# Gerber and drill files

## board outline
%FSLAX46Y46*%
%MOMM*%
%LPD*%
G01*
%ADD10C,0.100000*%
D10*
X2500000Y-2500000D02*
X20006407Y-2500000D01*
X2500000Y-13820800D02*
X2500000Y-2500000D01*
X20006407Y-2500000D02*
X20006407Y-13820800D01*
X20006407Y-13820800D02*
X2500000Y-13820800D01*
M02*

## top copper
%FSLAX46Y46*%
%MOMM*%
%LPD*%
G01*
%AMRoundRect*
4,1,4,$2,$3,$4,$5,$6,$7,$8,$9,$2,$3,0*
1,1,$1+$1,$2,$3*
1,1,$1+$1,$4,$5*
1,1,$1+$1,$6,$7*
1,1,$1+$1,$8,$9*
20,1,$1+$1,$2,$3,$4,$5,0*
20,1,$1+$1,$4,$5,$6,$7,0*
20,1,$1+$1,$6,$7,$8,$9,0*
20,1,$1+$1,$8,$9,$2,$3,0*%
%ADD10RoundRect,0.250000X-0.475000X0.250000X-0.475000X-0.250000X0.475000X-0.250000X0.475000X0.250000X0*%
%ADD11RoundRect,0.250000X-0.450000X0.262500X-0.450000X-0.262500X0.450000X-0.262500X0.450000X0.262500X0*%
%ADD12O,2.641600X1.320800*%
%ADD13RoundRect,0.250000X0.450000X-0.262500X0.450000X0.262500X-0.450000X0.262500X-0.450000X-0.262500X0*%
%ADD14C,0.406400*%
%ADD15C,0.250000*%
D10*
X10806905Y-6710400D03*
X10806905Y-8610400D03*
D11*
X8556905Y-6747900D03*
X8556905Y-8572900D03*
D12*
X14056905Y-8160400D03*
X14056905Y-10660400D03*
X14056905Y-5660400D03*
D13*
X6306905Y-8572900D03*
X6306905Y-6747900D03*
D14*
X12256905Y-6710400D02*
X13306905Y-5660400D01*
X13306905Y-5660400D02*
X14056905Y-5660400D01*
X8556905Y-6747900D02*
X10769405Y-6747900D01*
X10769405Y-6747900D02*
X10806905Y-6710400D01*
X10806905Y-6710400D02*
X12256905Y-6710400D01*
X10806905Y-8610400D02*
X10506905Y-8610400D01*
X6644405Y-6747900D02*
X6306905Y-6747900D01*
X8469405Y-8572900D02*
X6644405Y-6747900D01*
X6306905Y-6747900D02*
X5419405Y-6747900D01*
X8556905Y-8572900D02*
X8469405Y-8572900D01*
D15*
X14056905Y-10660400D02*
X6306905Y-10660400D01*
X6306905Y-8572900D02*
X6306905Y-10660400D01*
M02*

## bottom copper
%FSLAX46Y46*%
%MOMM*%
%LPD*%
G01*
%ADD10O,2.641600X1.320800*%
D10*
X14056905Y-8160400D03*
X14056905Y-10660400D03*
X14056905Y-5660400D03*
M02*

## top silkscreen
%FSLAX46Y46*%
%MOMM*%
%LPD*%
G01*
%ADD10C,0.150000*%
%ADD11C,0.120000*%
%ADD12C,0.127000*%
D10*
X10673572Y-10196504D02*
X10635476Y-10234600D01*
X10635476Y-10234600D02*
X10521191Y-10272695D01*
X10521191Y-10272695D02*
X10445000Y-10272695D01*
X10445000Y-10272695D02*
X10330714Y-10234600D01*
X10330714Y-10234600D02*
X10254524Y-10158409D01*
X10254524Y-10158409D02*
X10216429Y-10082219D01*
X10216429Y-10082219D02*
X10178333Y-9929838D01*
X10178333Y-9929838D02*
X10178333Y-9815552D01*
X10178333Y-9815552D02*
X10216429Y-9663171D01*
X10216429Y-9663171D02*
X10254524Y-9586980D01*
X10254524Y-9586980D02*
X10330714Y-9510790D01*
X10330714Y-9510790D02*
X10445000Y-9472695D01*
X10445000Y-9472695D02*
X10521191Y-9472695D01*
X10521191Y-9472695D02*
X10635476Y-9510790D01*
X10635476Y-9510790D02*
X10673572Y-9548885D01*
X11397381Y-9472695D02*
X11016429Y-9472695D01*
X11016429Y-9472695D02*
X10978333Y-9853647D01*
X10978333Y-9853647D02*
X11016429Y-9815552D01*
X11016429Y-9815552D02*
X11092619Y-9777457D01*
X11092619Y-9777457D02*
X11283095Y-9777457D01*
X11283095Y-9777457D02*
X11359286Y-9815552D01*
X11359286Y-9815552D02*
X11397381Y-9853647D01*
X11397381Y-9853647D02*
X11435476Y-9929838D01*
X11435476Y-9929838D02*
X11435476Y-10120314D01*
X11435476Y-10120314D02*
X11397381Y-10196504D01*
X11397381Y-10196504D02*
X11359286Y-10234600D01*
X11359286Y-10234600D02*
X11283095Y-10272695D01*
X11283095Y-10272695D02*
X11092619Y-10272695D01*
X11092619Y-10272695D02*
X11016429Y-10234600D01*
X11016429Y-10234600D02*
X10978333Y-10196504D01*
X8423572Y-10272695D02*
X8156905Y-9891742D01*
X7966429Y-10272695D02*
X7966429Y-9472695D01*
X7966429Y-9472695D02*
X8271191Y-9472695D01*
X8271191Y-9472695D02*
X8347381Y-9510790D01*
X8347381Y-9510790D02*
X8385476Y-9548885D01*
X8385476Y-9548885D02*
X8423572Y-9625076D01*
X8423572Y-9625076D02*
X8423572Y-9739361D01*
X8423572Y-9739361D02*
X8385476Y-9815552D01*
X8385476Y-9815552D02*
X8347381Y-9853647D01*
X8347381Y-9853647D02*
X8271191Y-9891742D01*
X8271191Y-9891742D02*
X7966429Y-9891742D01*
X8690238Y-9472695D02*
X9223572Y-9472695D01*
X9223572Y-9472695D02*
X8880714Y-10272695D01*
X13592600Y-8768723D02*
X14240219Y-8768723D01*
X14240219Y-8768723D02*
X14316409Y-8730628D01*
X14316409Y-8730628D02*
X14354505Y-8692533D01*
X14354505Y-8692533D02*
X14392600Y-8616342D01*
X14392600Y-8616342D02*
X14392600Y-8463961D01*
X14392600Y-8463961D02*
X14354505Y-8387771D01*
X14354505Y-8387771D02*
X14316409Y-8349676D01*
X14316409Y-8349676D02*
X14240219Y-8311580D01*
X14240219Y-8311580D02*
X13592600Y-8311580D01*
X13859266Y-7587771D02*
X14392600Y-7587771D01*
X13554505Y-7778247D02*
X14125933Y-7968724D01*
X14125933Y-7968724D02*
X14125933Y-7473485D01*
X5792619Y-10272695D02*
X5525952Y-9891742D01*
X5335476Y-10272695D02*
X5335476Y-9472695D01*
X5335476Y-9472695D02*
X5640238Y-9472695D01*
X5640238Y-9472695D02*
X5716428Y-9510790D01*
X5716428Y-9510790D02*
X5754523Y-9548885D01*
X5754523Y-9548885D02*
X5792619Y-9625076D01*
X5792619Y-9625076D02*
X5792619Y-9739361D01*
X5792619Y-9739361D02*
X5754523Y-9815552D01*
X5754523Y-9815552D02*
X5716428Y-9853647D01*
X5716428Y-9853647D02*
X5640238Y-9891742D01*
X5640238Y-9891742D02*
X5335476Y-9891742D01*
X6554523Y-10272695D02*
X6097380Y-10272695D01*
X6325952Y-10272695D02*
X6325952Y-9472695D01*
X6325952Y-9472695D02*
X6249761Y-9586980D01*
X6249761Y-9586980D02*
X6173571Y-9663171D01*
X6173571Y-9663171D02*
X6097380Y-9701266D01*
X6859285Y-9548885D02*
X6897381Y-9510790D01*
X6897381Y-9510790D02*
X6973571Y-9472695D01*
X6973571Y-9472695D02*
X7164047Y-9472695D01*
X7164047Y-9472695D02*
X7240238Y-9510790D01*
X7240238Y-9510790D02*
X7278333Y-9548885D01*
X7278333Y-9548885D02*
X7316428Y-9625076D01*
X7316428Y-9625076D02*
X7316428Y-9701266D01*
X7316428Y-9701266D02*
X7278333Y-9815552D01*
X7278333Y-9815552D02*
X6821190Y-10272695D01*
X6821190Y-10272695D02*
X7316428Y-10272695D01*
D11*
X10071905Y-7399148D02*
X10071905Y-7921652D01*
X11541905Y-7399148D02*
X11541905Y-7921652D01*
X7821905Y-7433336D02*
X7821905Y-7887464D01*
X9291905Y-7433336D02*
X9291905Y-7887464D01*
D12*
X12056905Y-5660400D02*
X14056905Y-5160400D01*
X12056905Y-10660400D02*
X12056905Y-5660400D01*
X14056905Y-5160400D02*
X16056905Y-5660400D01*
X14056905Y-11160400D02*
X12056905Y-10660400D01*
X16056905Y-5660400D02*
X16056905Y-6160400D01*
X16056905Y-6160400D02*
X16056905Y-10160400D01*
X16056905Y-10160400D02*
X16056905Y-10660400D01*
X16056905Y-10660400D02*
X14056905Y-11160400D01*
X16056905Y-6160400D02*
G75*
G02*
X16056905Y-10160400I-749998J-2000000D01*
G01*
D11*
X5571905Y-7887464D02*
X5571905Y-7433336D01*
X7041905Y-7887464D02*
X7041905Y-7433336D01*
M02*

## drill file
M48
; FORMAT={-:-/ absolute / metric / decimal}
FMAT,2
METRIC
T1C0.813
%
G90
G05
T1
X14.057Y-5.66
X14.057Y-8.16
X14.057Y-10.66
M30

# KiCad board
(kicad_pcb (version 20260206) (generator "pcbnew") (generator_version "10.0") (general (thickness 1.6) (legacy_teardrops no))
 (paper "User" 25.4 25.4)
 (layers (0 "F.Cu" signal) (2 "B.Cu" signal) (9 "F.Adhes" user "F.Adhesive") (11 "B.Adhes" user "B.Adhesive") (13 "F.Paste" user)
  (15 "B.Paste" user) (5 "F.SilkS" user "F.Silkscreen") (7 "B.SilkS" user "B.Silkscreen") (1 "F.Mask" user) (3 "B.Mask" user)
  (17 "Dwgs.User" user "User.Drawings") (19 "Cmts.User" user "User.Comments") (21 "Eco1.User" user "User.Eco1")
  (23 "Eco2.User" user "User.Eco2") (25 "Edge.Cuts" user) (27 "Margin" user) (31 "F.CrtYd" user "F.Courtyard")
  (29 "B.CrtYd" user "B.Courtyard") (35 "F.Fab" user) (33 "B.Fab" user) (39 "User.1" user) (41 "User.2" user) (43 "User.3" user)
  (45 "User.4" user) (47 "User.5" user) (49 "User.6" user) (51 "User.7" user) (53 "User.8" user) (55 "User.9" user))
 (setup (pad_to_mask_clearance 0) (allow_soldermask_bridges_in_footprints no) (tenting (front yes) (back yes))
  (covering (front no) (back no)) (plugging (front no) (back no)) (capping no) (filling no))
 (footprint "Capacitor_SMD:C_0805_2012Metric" (layer "F.Cu") (at 10.806905 7.6604 -90)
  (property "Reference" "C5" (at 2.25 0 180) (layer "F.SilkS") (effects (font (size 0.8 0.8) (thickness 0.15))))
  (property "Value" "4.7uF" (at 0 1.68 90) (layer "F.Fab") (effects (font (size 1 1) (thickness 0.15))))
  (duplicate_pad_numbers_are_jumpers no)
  (fp_line (start -0.261252 0.735) (end 0.261252 0.735) (stroke (width 0.12) (type solid)) (layer "F.SilkS"))
  (fp_line (start -0.261252 -0.735) (end 0.261252 -0.735) (stroke (width 0.12) (type solid)) (layer "F.SilkS"))
  (pad "1" smd roundrect (at -0.95 0 270) (size 1 1.45) (layers "F.Cu" "F.Mask" "F.Paste") (roundrect_rratio 0.25) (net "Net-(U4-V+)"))
  (pad "2" smd roundrect (at 0.95 0 270) (size 1 1.45) (layers "F.Cu" "F.Mask" "F.Paste") (roundrect_rratio 0.25) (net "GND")))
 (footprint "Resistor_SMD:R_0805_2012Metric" (layer "F.Cu") (at 8.556905 7.6604 -90)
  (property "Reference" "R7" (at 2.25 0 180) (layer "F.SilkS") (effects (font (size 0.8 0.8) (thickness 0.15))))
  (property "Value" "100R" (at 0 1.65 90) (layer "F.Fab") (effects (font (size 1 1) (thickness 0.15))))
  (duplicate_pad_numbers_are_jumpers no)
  (fp_line (start -0.227064 0.735) (end 0.227064 0.735) (stroke (width 0.12) (type solid)) (layer "F.SilkS"))
  (fp_line (start -0.227064 -0.735) (end 0.227064 -0.735) (stroke (width 0.12) (type solid)) (layer "F.SilkS"))
  (pad "1" smd roundrect (at -0.9125 0 270) (size 1.025 1.4) (layers "F.Cu" "F.Mask" "F.Paste") (roundrect_rratio 0.243902439)
   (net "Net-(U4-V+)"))
  (pad "2" smd roundrect (at 0.9125 0 270) (size 1.025 1.4) (layers "F.Cu" "F.Mask" "F.Paste") (roundrect_rratio 0.243902439) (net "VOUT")))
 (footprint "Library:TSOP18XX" (layer "F.Cu") (at 14.030305 8.1592 90)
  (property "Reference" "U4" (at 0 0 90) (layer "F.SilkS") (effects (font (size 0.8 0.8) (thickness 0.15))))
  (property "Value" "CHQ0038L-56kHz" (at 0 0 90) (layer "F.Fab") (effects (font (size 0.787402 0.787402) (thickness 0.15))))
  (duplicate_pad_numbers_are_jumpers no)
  (fp_line (start 2.4988 -1.9734) (end 2.9988 0.0266) (stroke (width 0.127) (type solid)) (layer "F.SilkS"))
  (fp_line (start -2.5012 -1.9734) (end 2.4988 -1.9734) (stroke (width 0.127) (type solid)) (layer "F.SilkS"))
  (fp_line (start 2.9988 0.0266) (end 2.4988 2.0266) (stroke (width 0.127) (type solid)) (layer "F.SilkS"))
  (fp_line (start -3.0012 0.0266) (end -2.5012 -1.9734) (stroke (width 0.127) (type solid)) (layer "F.SilkS"))
  (fp_line (start 2.4988 2.0266) (end 1.9988 2.0266) (stroke (width 0.127) (type solid)) (layer "F.SilkS"))
  (fp_line (start 1.9988 2.0266) (end -2.0012 2.0266) (stroke (width 0.127) (type solid)) (layer "F.SilkS"))
  (fp_line (start -2.0012 2.0266) (end -2.5012 2.0266) (stroke (width 0.127) (type solid)) (layer "F.SilkS"))
  (fp_line (start -2.5012 2.0266) (end -3.0012 0.0266) (stroke (width 0.127) (type solid)) (layer "F.SilkS"))
  (fp_arc (start 1.9988 2.0266) (mid -0.0012 3.412602) (end -2.0012 2.0266) (stroke (width 0.127) (type solid)) (layer "F.SilkS"))
  (pad "GND" thru_hole oval (at -0.0012 0.0266 90) (size 1.3208 2.6416) (drill 0.8128) (layers "*.Cu" "*.Mask") (remove_unused_layers no)
   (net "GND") (solder_mask_margin 0.102))
  (pad "OUT" thru_hole oval (at -2.5012 0.0266 90) (size 1.3208 2.6416) (drill 0.8128) (layers "*.Cu" "*.Mask") (remove_unused_layers no)
   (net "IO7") (solder_mask_margin 0.102))
  (pad "VCC" thru_hole oval (at 2.4988 0.0266 90) (size 1.3208 2.6416) (drill 0.8128) (layers "*.Cu" "*.Mask") (remove_unused_layers no)
   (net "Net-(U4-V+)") (solder_mask_margin 0.102)))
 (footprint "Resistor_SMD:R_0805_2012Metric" (layer "F.Cu") (at 6.306905 7.6604 90)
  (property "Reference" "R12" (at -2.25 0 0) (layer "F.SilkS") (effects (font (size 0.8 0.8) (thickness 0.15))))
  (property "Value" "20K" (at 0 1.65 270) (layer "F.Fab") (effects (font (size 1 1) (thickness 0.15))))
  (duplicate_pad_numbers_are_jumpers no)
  (fp_line (start -0.227064 -0.735) (end 0.227064 -0.735) (stroke (width 0.12) (type solid)) (layer "F.SilkS"))
  (fp_line (start -0.227064 0.735) (end 0.227064 0.735) (stroke (width 0.12) (type solid)) (layer "F.SilkS"))
  (pad "1" smd roundrect (at -0.9125 0 90) (size 1.025 1.4) (layers "F.Cu" "F.Mask" "F.Paste") (roundrect_rratio 0.243902439) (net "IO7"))
  (pad "2" smd roundrect (at 0.9125 0 90) (size 1.025 1.4) (layers "F.Cu" "F.Mask" "F.Paste") (roundrect_rratio 0.243902439) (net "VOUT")))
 (gr_line (start 2.5 2.5) (end 20.006407 2.5) (stroke (width 0.1) (type default)) (layer "Edge.Cuts"))
 (gr_line (start 2.5 13.8208) (end 2.5 2.5) (stroke (width 0.1) (type default)) (layer "Edge.Cuts"))
 (gr_line (start 20.006407 2.5) (end 20.006407 13.8208) (stroke (width 0.1) (type default)) (layer "Edge.Cuts"))
 (gr_line (start 20.006407 13.8208) (end 2.5 13.8208) (stroke (width 0.1) (type default)) (layer "Edge.Cuts"))
 (segment (start 12.256905 6.7104) (end 13.306905 5.6604) (width 0.4064) (layer "F.Cu") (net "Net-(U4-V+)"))
 (segment (start 13.306905 5.6604) (end 14.056905 5.6604) (width 0.4064) (layer "F.Cu") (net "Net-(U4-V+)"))
 (segment (start 8.556905 6.7479) (end 10.769405 6.7479) (width 0.4064) (layer "F.Cu") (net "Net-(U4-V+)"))
 (segment (start 10.769405 6.7479) (end 10.806905 6.7104) (width 0.4064) (layer "F.Cu") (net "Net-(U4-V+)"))
 (segment (start 10.806905 6.7104) (end 12.256905 6.7104) (width 0.4064) (layer "F.Cu") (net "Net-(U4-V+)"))
 (segment (start 10.806905 8.6104) (end 10.506905 8.6104) (width 0.4064) (layer "F.Cu") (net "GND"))
 (segment (start 6.644405 6.7479) (end 6.306905 6.7479) (width 0.4064) (layer "F.Cu") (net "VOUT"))
 (segment (start 8.469405 8.5729) (end 6.644405 6.7479) (width 0.4064) (layer "F.Cu") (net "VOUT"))
 (segment (start 6.306905 6.7479) (end 5.419405 6.7479) (width 0.4064) (layer "F.Cu") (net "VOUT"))
 (segment (start 8.556905 8.5729) (end 8.469405 8.5729) (width 0.4064) (layer "F.Cu") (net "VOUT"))
 (segment (start 14.056905 10.6604) (end 6.306905 10.6604) (width 0.25) (layer "F.Cu") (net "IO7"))
 (segment (start 6.306905 8.5729) (end 6.306905 10.6604) (width 0.25) (layer "F.Cu") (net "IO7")))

